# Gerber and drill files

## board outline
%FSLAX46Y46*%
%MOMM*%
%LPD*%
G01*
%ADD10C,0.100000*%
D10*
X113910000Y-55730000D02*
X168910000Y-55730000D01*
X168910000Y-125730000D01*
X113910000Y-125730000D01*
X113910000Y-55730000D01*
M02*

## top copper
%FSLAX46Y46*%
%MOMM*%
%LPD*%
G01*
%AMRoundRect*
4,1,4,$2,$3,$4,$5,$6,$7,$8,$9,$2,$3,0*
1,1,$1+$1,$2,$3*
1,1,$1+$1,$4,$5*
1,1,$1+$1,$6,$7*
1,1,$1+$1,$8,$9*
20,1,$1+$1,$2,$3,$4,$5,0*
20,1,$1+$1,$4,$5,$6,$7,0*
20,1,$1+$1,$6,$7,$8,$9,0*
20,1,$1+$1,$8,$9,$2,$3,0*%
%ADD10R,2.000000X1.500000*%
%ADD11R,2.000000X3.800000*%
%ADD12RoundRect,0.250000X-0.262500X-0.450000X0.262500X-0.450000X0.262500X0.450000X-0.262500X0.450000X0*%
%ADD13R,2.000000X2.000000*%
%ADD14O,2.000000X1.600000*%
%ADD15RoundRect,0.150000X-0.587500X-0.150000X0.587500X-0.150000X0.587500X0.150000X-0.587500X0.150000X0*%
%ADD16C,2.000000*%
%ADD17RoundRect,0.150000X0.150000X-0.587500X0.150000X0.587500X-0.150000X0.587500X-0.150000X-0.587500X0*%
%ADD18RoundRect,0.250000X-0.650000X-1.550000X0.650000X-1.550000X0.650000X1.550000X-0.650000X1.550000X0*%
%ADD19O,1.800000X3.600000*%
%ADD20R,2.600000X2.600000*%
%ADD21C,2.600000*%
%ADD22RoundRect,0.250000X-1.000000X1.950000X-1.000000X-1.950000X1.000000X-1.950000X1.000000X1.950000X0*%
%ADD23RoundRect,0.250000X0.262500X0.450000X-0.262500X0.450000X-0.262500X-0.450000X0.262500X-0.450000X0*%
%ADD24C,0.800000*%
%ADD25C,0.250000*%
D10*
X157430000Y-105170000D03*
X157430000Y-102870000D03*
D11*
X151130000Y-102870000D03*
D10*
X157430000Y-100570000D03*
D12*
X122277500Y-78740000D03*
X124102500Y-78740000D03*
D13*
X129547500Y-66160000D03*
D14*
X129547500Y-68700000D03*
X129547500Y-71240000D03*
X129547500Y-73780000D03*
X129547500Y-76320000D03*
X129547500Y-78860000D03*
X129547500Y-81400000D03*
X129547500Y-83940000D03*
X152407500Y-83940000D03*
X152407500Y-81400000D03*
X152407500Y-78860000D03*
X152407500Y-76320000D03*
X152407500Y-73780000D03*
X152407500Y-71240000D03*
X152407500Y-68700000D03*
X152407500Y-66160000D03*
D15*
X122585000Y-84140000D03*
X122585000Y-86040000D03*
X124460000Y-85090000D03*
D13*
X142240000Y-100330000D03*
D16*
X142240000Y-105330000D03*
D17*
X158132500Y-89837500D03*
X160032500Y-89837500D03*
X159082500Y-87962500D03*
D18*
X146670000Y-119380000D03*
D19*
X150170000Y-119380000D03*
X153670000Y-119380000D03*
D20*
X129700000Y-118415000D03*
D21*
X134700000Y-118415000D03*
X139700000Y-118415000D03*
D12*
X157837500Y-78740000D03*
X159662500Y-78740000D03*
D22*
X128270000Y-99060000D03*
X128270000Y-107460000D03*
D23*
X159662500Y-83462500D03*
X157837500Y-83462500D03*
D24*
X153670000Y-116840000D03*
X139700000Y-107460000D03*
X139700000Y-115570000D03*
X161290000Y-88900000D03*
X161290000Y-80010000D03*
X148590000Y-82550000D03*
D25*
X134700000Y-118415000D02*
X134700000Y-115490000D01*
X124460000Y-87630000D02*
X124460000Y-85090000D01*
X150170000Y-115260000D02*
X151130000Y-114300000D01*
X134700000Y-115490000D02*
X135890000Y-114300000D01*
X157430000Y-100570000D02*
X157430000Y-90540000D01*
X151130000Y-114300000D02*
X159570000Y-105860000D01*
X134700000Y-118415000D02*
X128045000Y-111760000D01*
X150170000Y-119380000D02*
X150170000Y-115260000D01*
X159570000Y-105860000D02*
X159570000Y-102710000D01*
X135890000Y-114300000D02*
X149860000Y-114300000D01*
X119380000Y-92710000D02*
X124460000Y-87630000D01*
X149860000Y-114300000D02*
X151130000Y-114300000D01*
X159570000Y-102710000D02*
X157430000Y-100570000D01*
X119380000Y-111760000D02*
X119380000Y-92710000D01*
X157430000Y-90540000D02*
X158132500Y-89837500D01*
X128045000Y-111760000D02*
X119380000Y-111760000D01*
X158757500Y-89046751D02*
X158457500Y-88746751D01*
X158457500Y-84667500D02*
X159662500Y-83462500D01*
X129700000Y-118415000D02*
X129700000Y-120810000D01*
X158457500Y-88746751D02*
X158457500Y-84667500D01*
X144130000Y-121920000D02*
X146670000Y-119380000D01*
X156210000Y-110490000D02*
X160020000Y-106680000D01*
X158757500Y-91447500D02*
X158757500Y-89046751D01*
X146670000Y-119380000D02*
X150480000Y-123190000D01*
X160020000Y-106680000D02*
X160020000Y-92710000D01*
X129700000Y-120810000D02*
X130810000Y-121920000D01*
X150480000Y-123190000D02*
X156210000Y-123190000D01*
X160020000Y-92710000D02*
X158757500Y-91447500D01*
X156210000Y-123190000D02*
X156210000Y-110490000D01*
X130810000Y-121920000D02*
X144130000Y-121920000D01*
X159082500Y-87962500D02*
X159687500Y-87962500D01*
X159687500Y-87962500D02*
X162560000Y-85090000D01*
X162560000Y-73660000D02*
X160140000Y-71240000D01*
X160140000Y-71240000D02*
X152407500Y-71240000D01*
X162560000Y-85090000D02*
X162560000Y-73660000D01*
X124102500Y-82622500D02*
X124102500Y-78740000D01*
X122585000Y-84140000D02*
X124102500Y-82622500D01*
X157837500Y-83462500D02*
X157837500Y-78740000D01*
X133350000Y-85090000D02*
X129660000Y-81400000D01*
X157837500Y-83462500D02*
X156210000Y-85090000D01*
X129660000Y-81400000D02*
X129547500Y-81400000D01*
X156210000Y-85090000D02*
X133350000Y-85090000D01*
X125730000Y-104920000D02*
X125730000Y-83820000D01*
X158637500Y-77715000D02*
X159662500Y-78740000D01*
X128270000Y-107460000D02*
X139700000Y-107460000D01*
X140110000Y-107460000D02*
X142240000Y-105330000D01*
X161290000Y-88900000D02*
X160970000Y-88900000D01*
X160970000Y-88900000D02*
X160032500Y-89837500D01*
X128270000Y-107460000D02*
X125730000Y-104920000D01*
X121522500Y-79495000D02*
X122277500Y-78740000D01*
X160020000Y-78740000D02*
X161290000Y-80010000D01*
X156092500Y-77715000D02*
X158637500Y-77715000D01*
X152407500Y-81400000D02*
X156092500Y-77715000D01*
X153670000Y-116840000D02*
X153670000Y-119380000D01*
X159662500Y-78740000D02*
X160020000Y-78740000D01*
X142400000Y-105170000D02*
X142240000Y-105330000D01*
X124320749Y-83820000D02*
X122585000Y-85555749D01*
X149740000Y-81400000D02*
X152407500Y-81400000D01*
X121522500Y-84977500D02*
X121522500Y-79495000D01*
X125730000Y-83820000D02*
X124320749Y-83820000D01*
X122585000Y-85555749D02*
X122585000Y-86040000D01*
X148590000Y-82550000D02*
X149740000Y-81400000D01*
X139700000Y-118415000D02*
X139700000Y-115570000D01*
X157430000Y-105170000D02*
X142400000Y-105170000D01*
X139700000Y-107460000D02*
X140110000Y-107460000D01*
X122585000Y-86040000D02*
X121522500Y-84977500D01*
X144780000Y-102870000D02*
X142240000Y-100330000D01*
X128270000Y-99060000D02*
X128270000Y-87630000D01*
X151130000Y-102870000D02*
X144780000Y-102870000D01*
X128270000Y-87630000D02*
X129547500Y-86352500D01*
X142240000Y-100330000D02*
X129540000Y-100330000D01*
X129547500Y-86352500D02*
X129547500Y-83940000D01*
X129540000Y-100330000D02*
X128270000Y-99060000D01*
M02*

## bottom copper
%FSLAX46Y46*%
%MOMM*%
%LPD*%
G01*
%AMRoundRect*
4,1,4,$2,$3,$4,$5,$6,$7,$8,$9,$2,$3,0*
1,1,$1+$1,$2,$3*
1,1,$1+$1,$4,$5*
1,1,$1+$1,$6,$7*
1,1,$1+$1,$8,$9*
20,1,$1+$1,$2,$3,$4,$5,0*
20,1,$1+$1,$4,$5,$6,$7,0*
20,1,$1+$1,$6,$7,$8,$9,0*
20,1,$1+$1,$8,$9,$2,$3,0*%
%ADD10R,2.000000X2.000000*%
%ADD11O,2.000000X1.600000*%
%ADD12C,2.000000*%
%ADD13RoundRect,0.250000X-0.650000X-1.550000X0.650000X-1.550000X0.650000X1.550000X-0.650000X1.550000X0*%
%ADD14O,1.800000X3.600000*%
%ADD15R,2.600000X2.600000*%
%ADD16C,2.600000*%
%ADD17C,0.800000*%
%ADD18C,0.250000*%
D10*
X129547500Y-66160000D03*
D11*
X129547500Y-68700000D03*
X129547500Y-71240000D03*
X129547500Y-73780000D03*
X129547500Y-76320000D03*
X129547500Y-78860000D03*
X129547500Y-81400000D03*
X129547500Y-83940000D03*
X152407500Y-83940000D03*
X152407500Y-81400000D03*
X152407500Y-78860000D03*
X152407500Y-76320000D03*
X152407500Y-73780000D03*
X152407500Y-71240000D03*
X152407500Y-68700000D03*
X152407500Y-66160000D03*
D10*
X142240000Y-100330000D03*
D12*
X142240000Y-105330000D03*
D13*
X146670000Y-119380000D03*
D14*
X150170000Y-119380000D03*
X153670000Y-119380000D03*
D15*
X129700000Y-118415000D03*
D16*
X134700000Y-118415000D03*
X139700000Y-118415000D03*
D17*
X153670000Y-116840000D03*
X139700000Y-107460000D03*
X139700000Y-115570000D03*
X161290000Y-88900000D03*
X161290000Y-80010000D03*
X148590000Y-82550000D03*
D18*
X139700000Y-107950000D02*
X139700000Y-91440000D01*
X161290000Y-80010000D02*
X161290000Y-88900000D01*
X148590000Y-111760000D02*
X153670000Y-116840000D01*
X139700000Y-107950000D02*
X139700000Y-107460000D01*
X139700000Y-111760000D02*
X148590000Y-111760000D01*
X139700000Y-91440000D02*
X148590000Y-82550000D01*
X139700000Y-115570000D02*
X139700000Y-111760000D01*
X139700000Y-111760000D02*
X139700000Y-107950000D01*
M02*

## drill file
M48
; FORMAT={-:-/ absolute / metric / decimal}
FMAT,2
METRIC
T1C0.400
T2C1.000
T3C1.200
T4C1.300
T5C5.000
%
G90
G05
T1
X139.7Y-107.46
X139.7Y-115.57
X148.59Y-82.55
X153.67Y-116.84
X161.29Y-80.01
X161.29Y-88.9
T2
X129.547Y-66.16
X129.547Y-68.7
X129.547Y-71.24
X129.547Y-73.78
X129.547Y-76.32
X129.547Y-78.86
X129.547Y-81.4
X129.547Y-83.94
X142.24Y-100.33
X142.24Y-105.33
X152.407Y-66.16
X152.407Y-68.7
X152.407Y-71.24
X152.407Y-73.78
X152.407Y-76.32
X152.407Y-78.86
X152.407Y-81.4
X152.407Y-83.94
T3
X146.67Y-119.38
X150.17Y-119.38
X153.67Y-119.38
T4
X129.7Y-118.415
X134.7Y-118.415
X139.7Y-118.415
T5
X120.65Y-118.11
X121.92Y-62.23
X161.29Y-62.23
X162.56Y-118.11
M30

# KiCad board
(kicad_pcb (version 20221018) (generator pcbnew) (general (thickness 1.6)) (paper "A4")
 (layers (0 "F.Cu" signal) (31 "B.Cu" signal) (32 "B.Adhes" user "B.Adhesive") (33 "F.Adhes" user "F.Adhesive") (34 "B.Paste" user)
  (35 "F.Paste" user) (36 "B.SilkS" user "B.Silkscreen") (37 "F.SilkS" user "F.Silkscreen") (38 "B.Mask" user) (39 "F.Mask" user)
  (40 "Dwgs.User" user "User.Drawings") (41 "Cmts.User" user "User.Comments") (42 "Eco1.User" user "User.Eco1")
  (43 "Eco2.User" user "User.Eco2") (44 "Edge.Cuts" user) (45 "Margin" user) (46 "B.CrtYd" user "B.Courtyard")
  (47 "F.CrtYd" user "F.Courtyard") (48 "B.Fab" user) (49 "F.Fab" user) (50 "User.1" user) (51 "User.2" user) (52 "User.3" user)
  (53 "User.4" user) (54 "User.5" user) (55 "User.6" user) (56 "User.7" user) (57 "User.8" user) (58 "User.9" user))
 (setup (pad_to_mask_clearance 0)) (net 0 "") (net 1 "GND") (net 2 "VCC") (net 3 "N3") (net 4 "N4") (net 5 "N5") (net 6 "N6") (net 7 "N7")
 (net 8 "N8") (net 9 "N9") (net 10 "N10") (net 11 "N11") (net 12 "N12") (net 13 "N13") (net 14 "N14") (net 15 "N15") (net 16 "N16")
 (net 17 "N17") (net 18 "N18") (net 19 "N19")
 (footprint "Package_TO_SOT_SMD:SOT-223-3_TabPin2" (layer "F.Cu") (at 154.28 102.87 180)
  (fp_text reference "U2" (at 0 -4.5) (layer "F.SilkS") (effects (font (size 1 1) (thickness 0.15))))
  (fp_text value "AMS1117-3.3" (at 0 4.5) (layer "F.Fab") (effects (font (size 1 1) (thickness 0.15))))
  (pad "1" smd rect (at -3.15 -2.3 180) (size 2 1.5) (layers "F.Cu" "F.Paste" "F.Mask") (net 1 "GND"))
  (pad "2" smd rect (at -3.15 0 180) (size 2 1.5) (layers "F.Cu" "F.Paste" "F.Mask") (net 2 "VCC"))
  (pad "2" smd rect (at 3.15 0 180) (size 2 3.8) (layers "F.Cu" "F.Paste" "F.Mask") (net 2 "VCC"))
  (pad "3" smd rect (at -3.15 2.3 180) (size 2 1.5) (layers "F.Cu" "F.Paste" "F.Mask") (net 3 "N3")))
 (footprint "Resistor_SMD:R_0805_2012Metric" (layer "F.Cu") (at 123.19 78.74)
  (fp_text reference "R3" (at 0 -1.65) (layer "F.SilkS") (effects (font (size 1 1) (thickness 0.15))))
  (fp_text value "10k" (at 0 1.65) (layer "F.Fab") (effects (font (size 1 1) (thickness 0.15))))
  (pad "1" smd roundrect (at -0.9125 0) (size 1.025 1.4) (layers "F.Cu" "F.Paste" "F.Mask") (roundrect_rratio 0.243902439) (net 1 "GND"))
  (pad "2" smd roundrect (at 0.9125 0) (size 1.025 1.4) (layers "F.Cu" "F.Paste" "F.Mask") (roundrect_rratio 0.243902439) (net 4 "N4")))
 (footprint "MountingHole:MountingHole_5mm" (layer "F.Cu") (at 161.29 62.23)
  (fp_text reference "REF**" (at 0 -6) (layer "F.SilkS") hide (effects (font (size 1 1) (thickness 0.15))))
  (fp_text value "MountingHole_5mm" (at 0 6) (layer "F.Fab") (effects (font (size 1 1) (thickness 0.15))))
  (pad "" np_thru_hole circle (at 0 0) (size 5 5) (drill 5) (layers "*.Cu" "*.Mask")))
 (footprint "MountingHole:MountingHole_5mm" (layer "F.Cu") (at 162.56 118.11)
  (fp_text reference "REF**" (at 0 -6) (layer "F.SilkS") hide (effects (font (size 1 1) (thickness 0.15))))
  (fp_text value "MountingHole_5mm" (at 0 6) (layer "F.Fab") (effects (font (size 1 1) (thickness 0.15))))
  (pad "" np_thru_hole circle (at 0 0) (size 5 5) (drill 5) (layers "F&B.Cu" "*.Mask")))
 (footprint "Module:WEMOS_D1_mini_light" (layer "F.Cu") (at 129.5475 66.16)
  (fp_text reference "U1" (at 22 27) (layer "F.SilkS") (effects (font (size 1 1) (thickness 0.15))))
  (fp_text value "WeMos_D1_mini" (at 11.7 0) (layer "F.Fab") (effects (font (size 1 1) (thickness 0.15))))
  (pad "1" thru_hole rect (at 0 0) (size 2 2) (drill 1) (layers "*.Cu" "*.Mask") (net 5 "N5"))
  (pad "2" thru_hole oval (at 0 2.54) (size 2 1.6) (drill 1) (layers "*.Cu" "*.Mask") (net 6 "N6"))
  (pad "3" thru_hole oval (at 0 5.08) (size 2 1.6) (drill 1) (layers "*.Cu" "*.Mask") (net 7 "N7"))
  (pad "4" thru_hole oval (at 0 7.62) (size 2 1.6) (drill 1) (layers "*.Cu" "*.Mask") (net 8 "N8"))
  (pad "5" thru_hole oval (at 0 10.16) (size 2 1.6) (drill 1) (layers "*.Cu" "*.Mask") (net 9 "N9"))
  (pad "6" thru_hole oval (at 0 12.7) (size 2 1.6) (drill 1) (layers "*.Cu" "*.Mask") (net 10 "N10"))
  (pad "7" thru_hole oval (at 0 15.24) (size 2 1.6) (drill 1) (layers "*.Cu" "*.Mask") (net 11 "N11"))
  (pad "8" thru_hole oval (at 0 17.78) (size 2 1.6) (drill 1) (layers "*.Cu" "*.Mask") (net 2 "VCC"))
  (pad "9" thru_hole oval (at 22.86 17.78) (size 2 1.6) (drill 1) (layers "*.Cu" "*.Mask") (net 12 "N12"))
  (pad "10" thru_hole oval (at 22.86 15.24) (size 2 1.6) (drill 1) (layers "*.Cu" "*.Mask") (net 1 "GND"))
  (pad "11" thru_hole oval (at 22.86 12.7) (size 2 1.6) (drill 1) (layers "*.Cu" "*.Mask") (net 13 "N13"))
  (pad "12" thru_hole oval (at 22.86 10.16) (size 2 1.6) (drill 1) (layers "*.Cu" "*.Mask") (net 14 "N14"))
  (pad "13" thru_hole oval (at 22.86 7.62) (size 2 1.6) (drill 1) (layers "*.Cu" "*.Mask") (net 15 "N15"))
  (pad "14" thru_hole oval (at 22.86 5.08) (size 2 1.6) (drill 1) (layers "*.Cu" "*.Mask") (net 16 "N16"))
  (pad "15" thru_hole oval (at 22.86 2.54) (size 2 1.6) (drill 1) (layers "*.Cu" "*.Mask") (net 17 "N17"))
  (pad "16" thru_hole oval (at 22.86 0) (size 2 1.6) (drill 1) (layers "*.Cu" "*.Mask") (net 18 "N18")))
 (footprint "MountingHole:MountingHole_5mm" (layer "F.Cu") (at 120.65 118.11)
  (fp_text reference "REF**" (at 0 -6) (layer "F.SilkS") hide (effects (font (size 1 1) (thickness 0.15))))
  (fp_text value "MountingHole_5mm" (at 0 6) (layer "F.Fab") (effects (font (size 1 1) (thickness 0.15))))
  (pad "" np_thru_hole circle (at 0 0) (size 5 5) (drill 5) (layers "F&B.Cu" "*.Mask")))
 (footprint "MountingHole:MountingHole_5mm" (layer "F.Cu") (at 121.92 62.23)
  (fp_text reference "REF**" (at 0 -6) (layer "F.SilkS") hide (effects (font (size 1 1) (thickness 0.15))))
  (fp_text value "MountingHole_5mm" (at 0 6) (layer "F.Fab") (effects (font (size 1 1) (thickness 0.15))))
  (pad "" np_thru_hole circle (at 0 0) (size 5 5) (drill 5) (layers "F&B.Cu" "*.Mask")))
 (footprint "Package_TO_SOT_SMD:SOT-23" (layer "F.Cu") (at 123.5225 85.09)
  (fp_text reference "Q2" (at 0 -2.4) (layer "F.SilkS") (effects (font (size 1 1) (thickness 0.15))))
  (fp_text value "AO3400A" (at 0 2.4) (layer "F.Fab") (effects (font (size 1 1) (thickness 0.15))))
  (pad "1" smd roundrect (at -0.9375 -0.95) (size 1.475 0.6) (layers "F.Cu" "F.Paste" "F.Mask") (roundrect_rratio 0.25) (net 4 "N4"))
  (pad "2" smd roundrect (at -0.9375 0.95) (size 1.475 0.6) (layers "F.Cu" "F.Paste" "F.Mask") (roundrect_rratio 0.25) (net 1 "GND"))
  (pad "3" smd roundrect (at 0.9375 0) (size 1.475 0.6) (layers "F.Cu" "F.Paste" "F.Mask") (roundrect_rratio 0.25) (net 3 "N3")))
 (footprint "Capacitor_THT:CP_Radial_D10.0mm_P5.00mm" (layer "F.Cu") (at 142.24 100.33 -90)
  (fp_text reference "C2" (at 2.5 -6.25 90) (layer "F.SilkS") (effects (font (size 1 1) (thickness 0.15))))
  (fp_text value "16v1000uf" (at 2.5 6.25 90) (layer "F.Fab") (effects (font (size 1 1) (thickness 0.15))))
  (pad "1" thru_hole rect (at 0 0 270) (size 2 2) (drill 1) (layers "*.Cu" "*.Mask") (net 2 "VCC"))
  (pad "2" thru_hole circle (at 5 0 270) (size 2 2) (drill 1) (layers "*.Cu" "*.Mask") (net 1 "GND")))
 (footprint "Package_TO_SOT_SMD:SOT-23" (layer "F.Cu") (at 159.0825 88.9 90)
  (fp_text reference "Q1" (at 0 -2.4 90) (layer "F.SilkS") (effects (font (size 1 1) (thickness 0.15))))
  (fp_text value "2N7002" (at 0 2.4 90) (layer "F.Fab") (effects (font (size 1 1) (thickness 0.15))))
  (pad "1" smd roundrect (at -0.9375 -0.95 90) (size 1.475 0.6) (layers "F.Cu" "F.Paste" "F.Mask") (roundrect_rratio 0.25) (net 3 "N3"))
  (pad "2" smd roundrect (at -0.9375 0.95 90) (size 1.475 0.6) (layers "F.Cu" "F.Paste" "F.Mask") (roundrect_rratio 0.25) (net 1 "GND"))
  (pad "3" smd roundrect (at 0.9375 0 90) (size 1.475 0.6) (layers "F.Cu" "F.Paste" "F.Mask") (roundrect_rratio 0.25) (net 16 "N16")))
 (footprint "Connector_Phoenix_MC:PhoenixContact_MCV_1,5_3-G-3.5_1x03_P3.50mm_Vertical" (layer "F.Cu") (at 146.67 119.38)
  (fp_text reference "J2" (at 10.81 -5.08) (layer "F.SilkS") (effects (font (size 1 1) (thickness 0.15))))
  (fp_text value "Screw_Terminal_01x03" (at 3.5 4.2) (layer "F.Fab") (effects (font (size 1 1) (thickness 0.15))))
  (pad "1" thru_hole roundrect (at 0 0) (size 1.8 3.6) (drill 1.2) (layers "*.Cu" "*.Mask") (roundrect_rratio 0.1388888889) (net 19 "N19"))
  (pad "2" thru_hole oval (at 3.5 0) (size 1.8 3.6) (drill 1.2) (layers "*.Cu" "*.Mask") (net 3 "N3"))
  (pad "3" thru_hole oval (at 7 0) (size 1.8 3.6) (drill 1.2) (layers "*.Cu" "*.Mask") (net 1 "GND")))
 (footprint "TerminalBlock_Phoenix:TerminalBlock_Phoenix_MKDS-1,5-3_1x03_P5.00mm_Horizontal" (layer "F.Cu") (at 129.7 118.415)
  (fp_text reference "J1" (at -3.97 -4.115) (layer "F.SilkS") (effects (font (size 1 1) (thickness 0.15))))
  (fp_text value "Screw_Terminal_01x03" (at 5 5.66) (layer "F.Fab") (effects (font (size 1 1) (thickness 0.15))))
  (pad "1" thru_hole rect (at 0 0) (size 2.6 2.6) (drill 1.3) (layers "*.Cu" "*.Mask") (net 19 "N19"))
  (pad "2" thru_hole circle (at 5 0) (size 2.6 2.6) (drill 1.3) (layers "*.Cu" "*.Mask") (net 3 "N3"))
  (pad "3" thru_hole circle (at 10 0) (size 2.6 2.6) (drill 1.3) (layers "*.Cu" "*.Mask") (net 1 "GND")))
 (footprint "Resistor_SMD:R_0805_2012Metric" (layer "F.Cu") (at 158.75 78.74)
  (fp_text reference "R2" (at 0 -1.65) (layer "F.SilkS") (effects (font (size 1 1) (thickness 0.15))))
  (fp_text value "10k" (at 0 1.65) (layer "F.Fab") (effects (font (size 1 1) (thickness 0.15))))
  (pad "1" smd roundrect (at -0.9125 0) (size 1.025 1.4) (layers "F.Cu" "F.Paste" "F.Mask") (roundrect_rratio 0.243902439) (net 11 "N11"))
  (pad "2" smd roundrect (at 0.9125 0) (size 1.025 1.4) (layers "F.Cu" "F.Paste" "F.Mask") (roundrect_rratio 0.243902439) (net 1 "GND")))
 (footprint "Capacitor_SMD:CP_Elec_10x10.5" (layer "F.Cu") (at 128.27 103.26 -90)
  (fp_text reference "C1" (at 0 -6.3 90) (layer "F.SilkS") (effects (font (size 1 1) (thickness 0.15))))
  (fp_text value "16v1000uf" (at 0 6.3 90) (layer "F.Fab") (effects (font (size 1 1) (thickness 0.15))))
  (pad "1" smd roundrect (at -4.2 0 270) (size 4.4 2.5) (layers "F.Cu" "F.Paste" "F.Mask") (roundrect_rratio 0.1) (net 2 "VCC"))
  (pad "2" smd roundrect (at 4.2 0 270) (size 4.4 2.5) (layers "F.Cu" "F.Paste" "F.Mask") (roundrect_rratio 0.1) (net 1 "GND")))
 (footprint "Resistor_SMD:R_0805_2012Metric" (layer "F.Cu") (at 158.75 83.4625 180)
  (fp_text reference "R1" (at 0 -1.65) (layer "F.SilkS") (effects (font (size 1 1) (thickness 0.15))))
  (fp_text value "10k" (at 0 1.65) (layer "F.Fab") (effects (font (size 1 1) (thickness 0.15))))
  (pad "1" smd roundrect (at -0.9125 0 180) (size 1.025 1.4) (layers "F.Cu" "F.Paste" "F.Mask") (roundrect_rratio 0.243902439)
   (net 19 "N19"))
  (pad "2" smd roundrect (at 0.9125 0 180) (size 1.025 1.4) (layers "F.Cu" "F.Paste" "F.Mask") (roundrect_rratio 0.243902439) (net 11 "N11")))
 (gr_rect (start 113.91 55.73) (end 168.91 125.73) (stroke (width 0.1) (type default)) (fill none) (layer "Edge.Cuts"))
 (segment (start 134.7 118.415) (end 134.7 115.49) (width 0.25) (layer "F.Cu") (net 3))
 (segment (start 124.46 87.63) (end 124.46 85.09) (width 0.25) (layer "F.Cu") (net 3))
 (segment (start 150.17 115.26) (end 151.13 114.3) (width 0.25) (layer "F.Cu") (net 3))
 (segment (start 134.7 115.49) (end 135.89 114.3) (width 0.25) (layer "F.Cu") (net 3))
 (segment (start 157.43 100.57) (end 157.43 90.54) (width 0.25) (layer "F.Cu") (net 3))
 (segment (start 151.13 114.3) (end 159.57 105.86) (width 0.25) (layer "F.Cu") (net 3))
 (segment (start 134.7 118.415) (end 128.045 111.76) (width 0.25) (layer "F.Cu") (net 3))
 (segment (start 150.17 119.38) (end 150.17 115.26) (width 0.25) (layer "F.Cu") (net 3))
 (segment (start 159.57 105.86) (end 159.57 102.71) (width 0.25) (layer "F.Cu") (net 3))
 (segment (start 135.89 114.3) (end 149.86 114.3) (width 0.25) (layer "F.Cu") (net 3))
 (segment (start 119.38 92.71) (end 124.46 87.63) (width 0.25) (layer "F.Cu") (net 3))
 (segment (start 149.86 114.3) (end 151.13 114.3) (width 0.25) (layer "F.Cu") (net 3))
 (segment (start 159.57 102.71) (end 157.43 100.57) (width 0.25) (layer "F.Cu") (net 3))
 (segment (start 119.38 111.76) (end 119.38 92.71) (width 0.25) (layer "F.Cu") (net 3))
 (segment (start 157.43 90.54) (end 158.1325 89.8375) (width 0.25) (layer "F.Cu") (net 3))
 (segment (start 128.045 111.76) (end 119.38 111.76) (width 0.25) (layer "F.Cu") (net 3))
 (segment (start 158.7575 89.046751) (end 158.4575 88.746751) (width 0.25) (layer "F.Cu") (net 19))
 (segment (start 158.4575 84.6675) (end 159.6625 83.4625) (width 0.25) (layer "F.Cu") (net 19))
 (segment (start 129.7 118.415) (end 129.7 120.81) (width 0.25) (layer "F.Cu") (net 19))
 (segment (start 158.4575 88.746751) (end 158.4575 84.6675) (width 0.25) (layer "F.Cu") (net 19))
 (segment (start 144.13 121.92) (end 146.67 119.38) (width 0.25) (layer "F.Cu") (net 19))
 (segment (start 156.21 110.49) (end 160.02 106.68) (width 0.25) (layer "F.Cu") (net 19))
 (segment (start 158.7575 91.4475) (end 158.7575 89.046751) (width 0.25) (layer "F.Cu") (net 19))
 (segment (start 146.67 119.38) (end 150.48 123.19) (width 0.25) (layer "F.Cu") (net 19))
 (segment (start 160.02 106.68) (end 160.02 92.71) (width 0.25) (layer "F.Cu") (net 19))
 (segment (start 129.7 120.81) (end 130.81 121.92) (width 0.25) (layer "F.Cu") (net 19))
 (segment (start 150.48 123.19) (end 156.21 123.19) (width 0.25) (layer "F.Cu") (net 19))
 (segment (start 160.02 92.71) (end 158.7575 91.4475) (width 0.25) (layer "F.Cu") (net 19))
 (segment (start 156.21 123.19) (end 156.21 110.49) (width 0.25) (layer "F.Cu") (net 19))
 (segment (start 130.81 121.92) (end 144.13 121.92) (width 0.25) (layer "F.Cu") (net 19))
 (segment (start 159.0825 87.9625) (end 159.6875 87.9625) (width 0.25) (layer "F.Cu") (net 16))
 (segment (start 159.6875 87.9625) (end 162.56 85.09) (width 0.25) (layer "F.Cu") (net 16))
 (segment (start 162.56 73.66) (end 160.14 71.24) (width 0.25) (layer "F.Cu") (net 16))
 (segment (start 160.14 71.24) (end 152.4075 71.24) (width 0.25) (layer "F.Cu") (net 16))
 (segment (start 162.56 85.09) (end 162.56 73.66) (width 0.25) (layer "F.Cu") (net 16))
 (segment (start 124.1025 82.6225) (end 124.1025 78.74) (width 0.25) (layer "F.Cu") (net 4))
 (segment (start 122.585 84.14) (end 124.1025 82.6225) (width 0.25) (layer "F.Cu") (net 4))
 (segment (start 157.8375 83.4625) (end 157.8375 78.74) (width 0.25) (layer "F.Cu") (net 11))
 (segment (start 133.35 85.09) (end 129.66 81.4) (width 0.25) (layer "F.Cu") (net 11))
 (segment (start 157.8375 83.4625) (end 156.21 85.09) (width 0.25) (layer "F.Cu") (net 11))
 (segment (start 129.66 81.4) (end 129.5475 81.4) (width 0.25) (layer "F.Cu") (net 11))
 (segment (start 156.21 85.09) (end 133.35 85.09) (width 0.25) (layer "F.Cu") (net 11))
 (segment (start 125.73 104.92) (end 125.73 83.82) (width 0.25) (layer "F.Cu") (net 1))
 (segment (start 158.6375 77.715) (end 159.6625 78.74) (width 0.25) (layer "F.Cu") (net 1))
 (segment (start 128.27 107.46) (end 139.7 107.46) (width 0.25) (layer "F.Cu") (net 1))
 (segment (start 140.11 107.46) (end 142.24 105.33) (width 0.25) (layer "F.Cu") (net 1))
 (segment (start 161.29 88.9) (end 160.97 88.9) (width 0.25) (layer "F.Cu") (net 1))
 (segment (start 160.97 88.9) (end 160.0325 89.8375) (width 0.25) (layer "F.Cu") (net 1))
 (segment (start 128.27 107.46) (end 125.73 104.92) (width 0.25) (layer "F.Cu") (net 1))
 (segment (start 121.5225 79.495) (end 122.2775 78.74) (width 0.25) (layer "F.Cu") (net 1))
 (segment (start 160.02 78.74) (end 161.29 80.01) (width 0.25) (layer "F.Cu") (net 1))
 (segment (start 156.0925 77.715) (end 158.6375 77.715) (width 0.25) (layer "F.Cu") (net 1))
 (segment (start 152.4075 81.4) (end 156.0925 77.715) (width 0.25) (layer "F.Cu") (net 1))
 (segment (start 153.67 116.84) (end 153.67 119.38) (width 0.25) (layer "F.Cu") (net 1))
 (segment (start 159.6625 78.74) (end 160.02 78.74) (width 0.25) (layer "F.Cu") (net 1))
 (segment (start 142.4 105.17) (end 142.24 105.33) (width 0.25) (layer "F.Cu") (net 1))
 (segment (start 124.320749 83.82) (end 122.585 85.555749) (width 0.25) (layer "F.Cu") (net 1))
 (segment (start 149.74 81.4) (end 152.4075 81.4) (width 0.25) (layer "F.Cu") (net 1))
 (segment (start 121.5225 84.9775) (end 121.5225 79.495) (width 0.25) (layer "F.Cu") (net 1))
 (segment (start 125.73 83.82) (end 124.320749 83.82) (width 0.25) (layer "F.Cu") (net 1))
 (segment (start 122.585 85.555749) (end 122.585 86.04) (width 0.25) (layer "F.Cu") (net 1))
 (segment (start 148.59 82.55) (end 149.74 81.4) (width 0.25) (layer "F.Cu") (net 1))
 (segment (start 139.7 118.415) (end 139.7 115.57) (width 0.25) (layer "F.Cu") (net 1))
 (segment (start 157.43 105.17) (end 142.4 105.17) (width 0.25) (layer "F.Cu") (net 1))
 (segment (start 139.7 107.46) (end 140.11 107.46) (width 0.25) (layer "F.Cu") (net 1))
 (segment (start 122.585 86.04) (end 121.5225 84.9775) (width 0.25) (layer "F.Cu") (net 1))
 (via (at 153.67 116.84) (size 0.8) (drill 0.4) (layers "F.Cu" "B.Cu") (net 1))
 (via (at 139.7 107.46) (size 0.8) (drill 0.4) (layers "F.Cu" "B.Cu") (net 1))
 (via (at 139.7 115.57) (size 0.8) (drill 0.4) (layers "F.Cu" "B.Cu") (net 1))
 (via (at 161.29 88.9) (size 0.8) (drill 0.4) (layers "F.Cu" "B.Cu") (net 1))
 (via (at 161.29 80.01) (size 0.8) (drill 0.4) (layers "F.Cu" "B.Cu") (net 1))
 (via (at 148.59 82.55) (size 0.8) (drill 0.4) (layers "F.Cu" "B.Cu") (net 1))
 (segment (start 139.7 107.95) (end 139.7 91.44) (width 0.25) (layer "B.Cu") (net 1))
 (segment (start 161.29 80.01) (end 161.29 88.9) (width 0.25) (layer "B.Cu") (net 1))
 (segment (start 148.59 111.76) (end 153.67 116.84) (width 0.25) (layer "B.Cu") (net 1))
 (segment (start 139.7 107.95) (end 139.7 107.46) (width 0.25) (layer "B.Cu") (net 1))
 (segment (start 139.7 111.76) (end 148.59 111.76) (width 0.25) (layer "B.Cu") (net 1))
 (segment (start 139.7 91.44) (end 148.59 82.55) (width 0.25) (layer "B.Cu") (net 1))
 (segment (start 139.7 115.57) (end 139.7 111.76) (width 0.25) (layer "B.Cu") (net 1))
 (segment (start 139.7 111.76) (end 139.7 107.95) (width 0.25) (layer "B.Cu") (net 1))
 (segment (start 144.78 102.87) (end 142.24 100.33) (width 0.25) (layer "F.Cu") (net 2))
 (segment (start 128.27 99.06) (end 128.27 87.63) (width 0.25) (layer "F.Cu") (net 2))
 (segment (start 151.13 102.87) (end 144.78 102.87) (width 0.25) (layer "F.Cu") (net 2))
 (segment (start 128.27 87.63) (end 129.5475 86.3525) (width 0.25) (layer "F.Cu") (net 2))
 (segment (start 142.24 100.33) (end 129.54 100.33) (width 0.25) (layer "F.Cu") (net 2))
 (segment (start 129.5475 86.3525) (end 129.5475 83.94) (width 0.25) (layer "F.Cu") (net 2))
 (segment (start 129.54 100.33) (end 128.27 99.06) (width 0.25) (layer "F.Cu") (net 2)))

